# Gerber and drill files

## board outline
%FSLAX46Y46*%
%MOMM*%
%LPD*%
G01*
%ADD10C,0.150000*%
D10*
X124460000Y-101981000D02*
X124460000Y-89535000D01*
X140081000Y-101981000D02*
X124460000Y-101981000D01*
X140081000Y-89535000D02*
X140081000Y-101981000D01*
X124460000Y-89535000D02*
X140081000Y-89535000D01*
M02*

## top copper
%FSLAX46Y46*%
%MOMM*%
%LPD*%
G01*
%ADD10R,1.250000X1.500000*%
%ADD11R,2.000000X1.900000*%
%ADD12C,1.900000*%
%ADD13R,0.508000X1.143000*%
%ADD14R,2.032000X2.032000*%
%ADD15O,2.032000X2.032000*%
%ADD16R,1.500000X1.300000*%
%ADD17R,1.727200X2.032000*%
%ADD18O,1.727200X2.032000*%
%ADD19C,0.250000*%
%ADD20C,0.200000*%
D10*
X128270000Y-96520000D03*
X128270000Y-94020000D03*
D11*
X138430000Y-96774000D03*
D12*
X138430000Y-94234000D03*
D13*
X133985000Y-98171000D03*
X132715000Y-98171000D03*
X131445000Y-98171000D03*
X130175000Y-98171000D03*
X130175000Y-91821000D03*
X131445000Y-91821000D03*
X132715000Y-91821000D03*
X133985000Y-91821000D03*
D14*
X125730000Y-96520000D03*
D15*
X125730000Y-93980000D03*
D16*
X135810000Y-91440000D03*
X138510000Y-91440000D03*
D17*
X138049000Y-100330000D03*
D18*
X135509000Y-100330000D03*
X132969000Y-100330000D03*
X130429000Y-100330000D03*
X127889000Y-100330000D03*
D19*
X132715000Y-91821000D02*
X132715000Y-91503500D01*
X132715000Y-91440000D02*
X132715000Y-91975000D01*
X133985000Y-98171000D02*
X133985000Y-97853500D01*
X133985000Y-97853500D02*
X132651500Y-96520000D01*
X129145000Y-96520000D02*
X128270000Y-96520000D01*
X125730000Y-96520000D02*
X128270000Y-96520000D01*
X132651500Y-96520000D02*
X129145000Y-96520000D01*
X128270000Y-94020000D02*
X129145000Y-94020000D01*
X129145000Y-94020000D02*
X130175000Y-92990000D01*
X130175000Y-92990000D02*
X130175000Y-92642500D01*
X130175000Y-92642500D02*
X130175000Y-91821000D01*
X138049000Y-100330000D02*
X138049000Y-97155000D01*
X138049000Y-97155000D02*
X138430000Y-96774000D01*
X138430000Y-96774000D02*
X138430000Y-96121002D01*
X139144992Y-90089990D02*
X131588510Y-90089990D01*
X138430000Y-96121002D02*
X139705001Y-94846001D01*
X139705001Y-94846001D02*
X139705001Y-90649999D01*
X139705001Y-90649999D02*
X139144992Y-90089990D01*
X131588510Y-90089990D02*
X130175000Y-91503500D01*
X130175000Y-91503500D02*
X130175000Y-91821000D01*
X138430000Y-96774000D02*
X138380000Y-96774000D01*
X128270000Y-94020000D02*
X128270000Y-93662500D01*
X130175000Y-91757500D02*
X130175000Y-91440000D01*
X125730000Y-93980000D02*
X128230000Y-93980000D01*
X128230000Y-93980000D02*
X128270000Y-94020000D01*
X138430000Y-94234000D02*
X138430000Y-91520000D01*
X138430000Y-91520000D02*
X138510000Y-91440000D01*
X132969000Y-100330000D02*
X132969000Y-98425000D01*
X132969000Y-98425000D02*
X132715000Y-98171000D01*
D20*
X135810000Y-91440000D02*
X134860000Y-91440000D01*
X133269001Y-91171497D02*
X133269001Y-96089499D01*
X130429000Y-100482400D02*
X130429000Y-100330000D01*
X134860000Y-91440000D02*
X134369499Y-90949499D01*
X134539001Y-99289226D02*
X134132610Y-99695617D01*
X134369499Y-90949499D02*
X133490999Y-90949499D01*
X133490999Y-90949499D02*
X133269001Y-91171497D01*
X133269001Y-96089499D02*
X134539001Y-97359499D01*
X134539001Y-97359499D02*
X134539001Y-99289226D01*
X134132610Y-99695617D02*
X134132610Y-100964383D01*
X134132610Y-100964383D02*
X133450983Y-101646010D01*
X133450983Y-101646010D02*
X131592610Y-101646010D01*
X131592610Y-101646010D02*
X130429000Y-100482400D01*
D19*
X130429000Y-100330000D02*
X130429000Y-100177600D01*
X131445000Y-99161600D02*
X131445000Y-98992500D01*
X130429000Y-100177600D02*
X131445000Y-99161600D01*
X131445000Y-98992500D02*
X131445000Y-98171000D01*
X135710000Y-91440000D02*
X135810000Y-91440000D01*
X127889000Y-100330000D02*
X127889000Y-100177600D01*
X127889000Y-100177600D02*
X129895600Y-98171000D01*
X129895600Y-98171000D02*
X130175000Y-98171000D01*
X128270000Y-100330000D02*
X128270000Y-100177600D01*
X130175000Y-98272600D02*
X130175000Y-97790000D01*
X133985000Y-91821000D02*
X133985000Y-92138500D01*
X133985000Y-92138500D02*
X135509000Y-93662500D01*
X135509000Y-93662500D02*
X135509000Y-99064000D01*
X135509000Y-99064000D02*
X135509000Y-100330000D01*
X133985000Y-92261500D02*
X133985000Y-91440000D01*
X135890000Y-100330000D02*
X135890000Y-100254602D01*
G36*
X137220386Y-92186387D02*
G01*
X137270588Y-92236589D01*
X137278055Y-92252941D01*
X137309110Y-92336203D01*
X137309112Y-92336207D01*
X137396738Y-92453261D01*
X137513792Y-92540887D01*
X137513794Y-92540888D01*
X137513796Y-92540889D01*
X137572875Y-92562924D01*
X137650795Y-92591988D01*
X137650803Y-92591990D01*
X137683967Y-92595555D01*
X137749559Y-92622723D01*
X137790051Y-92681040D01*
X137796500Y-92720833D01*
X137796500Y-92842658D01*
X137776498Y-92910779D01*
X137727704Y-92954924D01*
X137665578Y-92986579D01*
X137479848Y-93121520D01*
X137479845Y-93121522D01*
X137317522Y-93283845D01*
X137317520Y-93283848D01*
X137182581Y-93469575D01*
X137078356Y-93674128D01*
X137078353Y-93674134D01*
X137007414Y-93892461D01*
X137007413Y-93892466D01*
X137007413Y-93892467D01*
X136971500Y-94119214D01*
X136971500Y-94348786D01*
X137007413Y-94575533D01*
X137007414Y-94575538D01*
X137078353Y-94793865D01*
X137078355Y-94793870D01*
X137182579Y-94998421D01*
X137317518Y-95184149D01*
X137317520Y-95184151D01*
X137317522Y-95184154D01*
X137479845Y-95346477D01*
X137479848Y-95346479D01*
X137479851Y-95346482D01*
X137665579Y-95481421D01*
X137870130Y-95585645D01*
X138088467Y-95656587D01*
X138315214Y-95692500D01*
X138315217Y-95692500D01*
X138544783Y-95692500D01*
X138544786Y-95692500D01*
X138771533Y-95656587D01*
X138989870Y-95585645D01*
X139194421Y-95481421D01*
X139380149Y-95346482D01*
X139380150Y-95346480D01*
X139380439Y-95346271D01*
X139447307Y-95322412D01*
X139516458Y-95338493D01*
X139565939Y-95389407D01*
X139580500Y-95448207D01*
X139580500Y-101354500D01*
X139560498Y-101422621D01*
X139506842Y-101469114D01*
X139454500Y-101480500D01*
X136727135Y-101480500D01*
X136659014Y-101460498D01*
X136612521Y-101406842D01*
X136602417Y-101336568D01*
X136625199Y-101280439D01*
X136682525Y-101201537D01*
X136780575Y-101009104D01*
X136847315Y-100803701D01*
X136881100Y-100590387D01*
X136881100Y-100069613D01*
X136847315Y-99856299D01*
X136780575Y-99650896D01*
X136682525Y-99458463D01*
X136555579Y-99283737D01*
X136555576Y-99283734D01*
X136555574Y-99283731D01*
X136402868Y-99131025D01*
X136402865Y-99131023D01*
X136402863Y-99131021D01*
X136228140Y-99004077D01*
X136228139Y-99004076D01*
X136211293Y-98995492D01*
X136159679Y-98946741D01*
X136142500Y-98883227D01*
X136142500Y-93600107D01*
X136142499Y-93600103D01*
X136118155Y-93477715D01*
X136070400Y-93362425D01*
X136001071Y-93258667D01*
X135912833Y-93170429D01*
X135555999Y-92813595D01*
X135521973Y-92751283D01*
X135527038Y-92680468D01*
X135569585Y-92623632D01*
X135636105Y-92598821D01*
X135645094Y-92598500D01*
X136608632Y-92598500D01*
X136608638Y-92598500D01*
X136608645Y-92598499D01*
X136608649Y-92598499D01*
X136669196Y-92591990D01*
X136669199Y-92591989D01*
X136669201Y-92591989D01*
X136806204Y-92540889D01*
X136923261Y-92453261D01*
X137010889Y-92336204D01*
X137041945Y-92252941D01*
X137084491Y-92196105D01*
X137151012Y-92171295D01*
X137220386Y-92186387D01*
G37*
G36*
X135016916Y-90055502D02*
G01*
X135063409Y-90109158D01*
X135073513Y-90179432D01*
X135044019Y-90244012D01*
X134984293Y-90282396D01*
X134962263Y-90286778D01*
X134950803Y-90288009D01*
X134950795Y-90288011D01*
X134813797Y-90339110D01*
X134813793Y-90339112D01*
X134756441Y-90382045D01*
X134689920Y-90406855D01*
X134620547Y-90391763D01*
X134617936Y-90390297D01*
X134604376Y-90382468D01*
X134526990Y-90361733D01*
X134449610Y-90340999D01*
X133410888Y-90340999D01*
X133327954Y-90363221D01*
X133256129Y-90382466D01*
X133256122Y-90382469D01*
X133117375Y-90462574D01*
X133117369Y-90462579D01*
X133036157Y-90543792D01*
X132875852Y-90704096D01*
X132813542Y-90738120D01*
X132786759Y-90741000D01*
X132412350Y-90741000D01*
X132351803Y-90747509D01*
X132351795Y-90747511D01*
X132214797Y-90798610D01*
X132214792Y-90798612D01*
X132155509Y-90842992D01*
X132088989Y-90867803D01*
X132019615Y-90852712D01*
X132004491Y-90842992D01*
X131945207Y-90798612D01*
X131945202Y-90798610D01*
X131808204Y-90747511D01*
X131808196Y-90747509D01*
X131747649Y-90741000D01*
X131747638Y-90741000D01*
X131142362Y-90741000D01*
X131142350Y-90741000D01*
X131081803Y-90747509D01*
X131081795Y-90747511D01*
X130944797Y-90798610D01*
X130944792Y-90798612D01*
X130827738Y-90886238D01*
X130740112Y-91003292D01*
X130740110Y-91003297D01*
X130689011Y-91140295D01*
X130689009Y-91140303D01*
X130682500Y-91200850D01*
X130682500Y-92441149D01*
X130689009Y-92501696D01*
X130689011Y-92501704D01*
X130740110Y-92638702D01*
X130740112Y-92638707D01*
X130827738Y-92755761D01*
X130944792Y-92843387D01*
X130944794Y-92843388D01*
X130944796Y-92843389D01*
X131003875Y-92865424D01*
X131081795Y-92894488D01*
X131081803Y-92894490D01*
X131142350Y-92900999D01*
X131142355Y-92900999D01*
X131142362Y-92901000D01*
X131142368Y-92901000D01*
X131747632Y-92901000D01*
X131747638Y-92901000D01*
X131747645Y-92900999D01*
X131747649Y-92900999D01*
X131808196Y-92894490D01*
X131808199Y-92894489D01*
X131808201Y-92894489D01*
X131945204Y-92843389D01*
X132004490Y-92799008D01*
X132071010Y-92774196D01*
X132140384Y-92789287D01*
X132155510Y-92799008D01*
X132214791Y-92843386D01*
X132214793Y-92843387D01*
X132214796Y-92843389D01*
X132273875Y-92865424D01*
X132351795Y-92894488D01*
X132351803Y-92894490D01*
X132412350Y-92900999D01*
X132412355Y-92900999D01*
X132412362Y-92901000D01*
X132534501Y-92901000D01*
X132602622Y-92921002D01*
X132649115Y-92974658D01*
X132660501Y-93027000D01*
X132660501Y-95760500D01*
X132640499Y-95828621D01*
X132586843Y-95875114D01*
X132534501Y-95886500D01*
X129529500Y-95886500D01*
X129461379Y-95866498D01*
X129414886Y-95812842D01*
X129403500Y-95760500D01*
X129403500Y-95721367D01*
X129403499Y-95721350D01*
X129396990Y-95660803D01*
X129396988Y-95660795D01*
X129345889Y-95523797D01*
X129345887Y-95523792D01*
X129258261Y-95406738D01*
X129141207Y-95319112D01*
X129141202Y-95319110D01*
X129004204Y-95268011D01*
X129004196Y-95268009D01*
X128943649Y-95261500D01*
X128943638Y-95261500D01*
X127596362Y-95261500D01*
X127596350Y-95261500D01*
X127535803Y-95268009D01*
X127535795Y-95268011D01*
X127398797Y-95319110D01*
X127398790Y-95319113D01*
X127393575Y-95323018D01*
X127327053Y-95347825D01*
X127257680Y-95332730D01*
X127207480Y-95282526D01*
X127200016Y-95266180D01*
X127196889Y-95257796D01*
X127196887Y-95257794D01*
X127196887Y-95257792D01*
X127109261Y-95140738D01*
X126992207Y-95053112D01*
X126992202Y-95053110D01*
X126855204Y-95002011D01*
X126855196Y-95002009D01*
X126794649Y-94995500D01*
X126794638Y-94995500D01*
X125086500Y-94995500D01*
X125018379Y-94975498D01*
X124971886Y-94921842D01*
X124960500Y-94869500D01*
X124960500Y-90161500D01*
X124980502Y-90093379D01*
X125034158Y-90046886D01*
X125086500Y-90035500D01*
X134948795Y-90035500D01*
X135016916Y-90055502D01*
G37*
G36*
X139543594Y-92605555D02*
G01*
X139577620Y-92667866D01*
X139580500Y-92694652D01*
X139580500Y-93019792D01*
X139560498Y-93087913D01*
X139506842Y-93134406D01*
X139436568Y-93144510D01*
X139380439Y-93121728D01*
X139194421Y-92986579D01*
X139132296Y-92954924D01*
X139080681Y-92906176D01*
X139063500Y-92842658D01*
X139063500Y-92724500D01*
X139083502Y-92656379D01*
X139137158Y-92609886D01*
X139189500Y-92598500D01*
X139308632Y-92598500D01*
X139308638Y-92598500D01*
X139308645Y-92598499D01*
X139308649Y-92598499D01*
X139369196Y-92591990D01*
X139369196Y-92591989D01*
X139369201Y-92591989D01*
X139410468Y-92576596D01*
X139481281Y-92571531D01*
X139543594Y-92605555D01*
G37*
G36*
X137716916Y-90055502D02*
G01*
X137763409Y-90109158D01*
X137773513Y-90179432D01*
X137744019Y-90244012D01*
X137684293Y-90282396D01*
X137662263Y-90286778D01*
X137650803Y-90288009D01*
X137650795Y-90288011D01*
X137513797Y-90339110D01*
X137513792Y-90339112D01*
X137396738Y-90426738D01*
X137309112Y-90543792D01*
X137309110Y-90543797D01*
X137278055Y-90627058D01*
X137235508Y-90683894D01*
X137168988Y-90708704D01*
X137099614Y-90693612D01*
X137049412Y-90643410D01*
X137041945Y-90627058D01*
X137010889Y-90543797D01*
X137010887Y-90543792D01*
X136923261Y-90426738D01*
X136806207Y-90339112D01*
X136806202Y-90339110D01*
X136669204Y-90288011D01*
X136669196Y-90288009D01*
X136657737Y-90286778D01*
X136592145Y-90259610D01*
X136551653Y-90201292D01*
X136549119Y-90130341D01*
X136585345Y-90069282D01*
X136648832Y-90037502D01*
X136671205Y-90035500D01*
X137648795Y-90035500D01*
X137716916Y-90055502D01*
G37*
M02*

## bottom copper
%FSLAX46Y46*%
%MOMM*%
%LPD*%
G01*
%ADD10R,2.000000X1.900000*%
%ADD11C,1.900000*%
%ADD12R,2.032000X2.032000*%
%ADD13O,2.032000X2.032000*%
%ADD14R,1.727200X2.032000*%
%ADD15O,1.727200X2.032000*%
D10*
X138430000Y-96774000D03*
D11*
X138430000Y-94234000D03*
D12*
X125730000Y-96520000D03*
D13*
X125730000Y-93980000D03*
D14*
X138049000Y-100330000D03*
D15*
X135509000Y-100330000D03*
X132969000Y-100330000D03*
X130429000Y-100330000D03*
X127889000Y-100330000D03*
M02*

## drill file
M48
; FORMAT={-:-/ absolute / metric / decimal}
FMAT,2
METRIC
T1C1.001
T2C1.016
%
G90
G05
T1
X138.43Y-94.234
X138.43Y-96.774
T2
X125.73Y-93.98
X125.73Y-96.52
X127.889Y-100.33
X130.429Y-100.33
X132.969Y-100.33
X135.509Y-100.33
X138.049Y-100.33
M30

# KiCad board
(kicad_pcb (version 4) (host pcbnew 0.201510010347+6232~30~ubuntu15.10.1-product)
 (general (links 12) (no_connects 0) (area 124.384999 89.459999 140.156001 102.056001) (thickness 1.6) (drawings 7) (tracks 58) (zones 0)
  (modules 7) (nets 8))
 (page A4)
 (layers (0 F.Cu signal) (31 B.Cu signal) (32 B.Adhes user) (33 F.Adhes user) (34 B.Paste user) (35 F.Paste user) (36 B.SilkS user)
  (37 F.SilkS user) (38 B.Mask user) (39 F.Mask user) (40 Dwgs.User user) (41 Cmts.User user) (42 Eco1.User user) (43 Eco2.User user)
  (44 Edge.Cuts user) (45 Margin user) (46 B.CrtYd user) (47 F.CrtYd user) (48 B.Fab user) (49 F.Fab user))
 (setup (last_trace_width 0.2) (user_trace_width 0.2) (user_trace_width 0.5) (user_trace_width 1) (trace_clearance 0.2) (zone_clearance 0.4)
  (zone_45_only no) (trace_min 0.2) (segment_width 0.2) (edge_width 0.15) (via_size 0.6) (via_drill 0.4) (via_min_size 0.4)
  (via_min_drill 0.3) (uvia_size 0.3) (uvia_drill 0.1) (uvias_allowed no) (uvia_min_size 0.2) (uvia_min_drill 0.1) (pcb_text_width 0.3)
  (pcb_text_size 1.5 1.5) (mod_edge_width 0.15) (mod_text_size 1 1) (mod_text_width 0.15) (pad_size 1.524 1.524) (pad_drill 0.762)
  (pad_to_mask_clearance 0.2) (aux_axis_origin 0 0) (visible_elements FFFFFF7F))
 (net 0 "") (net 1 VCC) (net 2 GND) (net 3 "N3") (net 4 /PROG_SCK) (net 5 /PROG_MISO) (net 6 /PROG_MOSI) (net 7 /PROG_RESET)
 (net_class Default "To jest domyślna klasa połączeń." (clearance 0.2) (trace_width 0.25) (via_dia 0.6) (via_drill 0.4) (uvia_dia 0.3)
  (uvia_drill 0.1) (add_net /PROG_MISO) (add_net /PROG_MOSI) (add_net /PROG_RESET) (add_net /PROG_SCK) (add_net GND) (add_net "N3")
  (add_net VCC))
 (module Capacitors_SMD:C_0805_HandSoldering (layer F.Cu) (at 128.27 95.27 90)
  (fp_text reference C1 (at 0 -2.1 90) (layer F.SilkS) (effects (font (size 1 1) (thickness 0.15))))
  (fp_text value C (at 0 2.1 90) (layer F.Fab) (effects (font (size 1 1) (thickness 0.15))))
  (pad 1 smd rect (at -1.25 0 90) (size 1.5 1.25) (layers F.Cu F.Paste F.Mask) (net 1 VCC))
  (pad 2 smd rect (at 1.25 0 90) (size 1.5 1.25) (layers F.Cu F.Paste F.Mask) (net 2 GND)))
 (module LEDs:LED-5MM (layer B.Cu) (at 138.43 96.774 90)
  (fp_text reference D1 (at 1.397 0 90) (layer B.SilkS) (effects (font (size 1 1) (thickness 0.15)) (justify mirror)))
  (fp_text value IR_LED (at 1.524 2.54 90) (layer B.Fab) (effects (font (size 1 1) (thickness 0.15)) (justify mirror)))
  (pad 1 thru_hole rect (at 0 0) (size 2 1.9) (drill 1.00076) (layers *.Cu *.Mask B.SilkS) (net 2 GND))
  (pad 2 thru_hole circle (at 2.54 0 90) (size 1.9 1.9) (drill 1.00076) (layers *.Cu *.Mask B.SilkS) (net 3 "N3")))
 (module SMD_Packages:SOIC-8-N (layer F.Cu) (at 132.08 94.996 180)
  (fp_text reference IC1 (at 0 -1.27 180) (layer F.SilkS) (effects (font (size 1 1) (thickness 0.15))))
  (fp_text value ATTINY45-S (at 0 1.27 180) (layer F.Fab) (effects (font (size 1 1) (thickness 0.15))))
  (pad 8 smd rect (at -1.905 -3.175 180) (size 0.508 1.143) (layers F.Cu F.Paste F.Mask) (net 1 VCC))
  (pad 7 smd rect (at -0.635 -3.175 180) (size 0.508 1.143) (layers F.Cu F.Paste F.Mask) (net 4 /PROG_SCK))
  (pad 6 smd rect (at 0.635 -3.175 180) (size 0.508 1.143) (layers F.Cu F.Paste F.Mask) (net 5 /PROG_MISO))
  (pad 5 smd rect (at 1.905 -3.175 180) (size 0.508 1.143) (layers F.Cu F.Paste F.Mask) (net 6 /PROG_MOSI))
  (pad 4 smd rect (at 1.905 3.175 180) (size 0.508 1.143) (layers F.Cu F.Paste F.Mask) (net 2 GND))
  (pad 3 smd rect (at 0.635 3.175 180) (size 0.508 1.143) (layers F.Cu F.Paste F.Mask))
  (pad 2 smd rect (at -0.635 3.175 180) (size 0.508 1.143) (layers F.Cu F.Paste F.Mask))
  (pad 1 smd rect (at -1.905 3.175 180) (size 0.508 1.143) (layers F.Cu F.Paste F.Mask) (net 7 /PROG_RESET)))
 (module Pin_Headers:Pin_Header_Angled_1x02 (layer F.Cu) (at 125.73 96.52 180)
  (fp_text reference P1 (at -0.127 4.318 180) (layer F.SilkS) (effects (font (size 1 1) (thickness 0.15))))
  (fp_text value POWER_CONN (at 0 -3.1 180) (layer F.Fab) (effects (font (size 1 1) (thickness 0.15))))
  (pad 1 thru_hole rect (at 0 0 180) (size 2.032 2.032) (drill 1.016) (layers *.Cu *.Mask F.SilkS) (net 1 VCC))
  (pad 2 thru_hole oval (at 0 2.54 180) (size 2.032 2.032) (drill 1.016) (layers *.Cu *.Mask F.SilkS) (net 2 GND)))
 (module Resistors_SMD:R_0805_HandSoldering (layer F.Cu) (at 137.16 91.44)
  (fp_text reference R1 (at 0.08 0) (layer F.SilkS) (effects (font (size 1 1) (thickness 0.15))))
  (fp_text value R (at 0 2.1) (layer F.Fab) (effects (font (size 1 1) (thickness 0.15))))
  (pad 1 smd rect (at -1.35 0) (size 1.5 1.3) (layers F.Cu F.Paste F.Mask) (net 5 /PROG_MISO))
  (pad 2 smd rect (at 1.35 0) (size 1.5 1.3) (layers F.Cu F.Paste F.Mask) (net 3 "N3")))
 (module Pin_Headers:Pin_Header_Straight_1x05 (layer F.Cu) (at 138.049 100.33 270)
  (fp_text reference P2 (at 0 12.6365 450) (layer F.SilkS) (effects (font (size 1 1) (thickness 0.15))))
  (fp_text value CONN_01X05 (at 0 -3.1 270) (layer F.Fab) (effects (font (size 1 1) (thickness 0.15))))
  (pad 1 thru_hole rect (at 0 0 270) (size 2.032 1.7272) (drill 1.016) (layers *.Cu *.Mask F.SilkS) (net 2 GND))
  (pad 2 thru_hole oval (at 0 2.54 270) (size 2.032 1.7272) (drill 1.016) (layers *.Cu *.Mask F.SilkS) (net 7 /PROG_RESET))
  (pad 3 thru_hole oval (at 0 5.08 270) (size 2.032 1.7272) (drill 1.016) (layers *.Cu *.Mask F.SilkS) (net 4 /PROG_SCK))
  (pad 4 thru_hole oval (at 0 7.62 270) (size 2.032 1.7272) (drill 1.016) (layers *.Cu *.Mask F.SilkS) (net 5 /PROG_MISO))
  (pad 5 thru_hole oval (at 0 10.16 270) (size 2.032 1.7272) (drill 1.016) (layers *.Cu *.Mask F.SilkS) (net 6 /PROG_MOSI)))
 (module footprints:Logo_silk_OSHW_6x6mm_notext (layer B.Cu) (at 129.794 92.202)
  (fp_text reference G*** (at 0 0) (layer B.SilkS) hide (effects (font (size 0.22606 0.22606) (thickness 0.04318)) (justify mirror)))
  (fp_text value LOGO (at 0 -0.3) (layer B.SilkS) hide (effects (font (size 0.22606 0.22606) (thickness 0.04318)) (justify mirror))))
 (gr_line (start 124.46 101.981) (end 124.46 89.535) (layer Edge.Cuts) (width 0.15))
 (gr_line (start 140.081 101.981) (end 124.46 101.981) (layer Edge.Cuts) (width 0.15))
 (gr_line (start 140.081 89.535) (end 140.081 101.981) (layer Edge.Cuts) (width 0.15))
 (gr_line (start 124.46 89.535) (end 140.081 89.535) (layer Edge.Cuts) (width 0.15))
 (segment (start 132.715 91.821) (end 132.715 91.5035) (width 0.25) (layer F.Cu) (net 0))
 (segment (start 132.715 91.44) (end 132.715 91.975) (width 0.25) (layer F.Cu) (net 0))
 (segment (start 133.985 98.171) (end 133.985 97.8535) (width 0.25) (layer F.Cu) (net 1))
 (segment (start 133.985 97.8535) (end 132.6515 96.52) (width 0.25) (layer F.Cu) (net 1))
 (segment (start 129.145 96.52) (end 128.27 96.52) (width 0.25) (layer F.Cu) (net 1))
 (segment (start 125.73 96.52) (end 128.27 96.52) (width 0.25) (layer F.Cu) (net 1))
 (segment (start 132.6515 96.52) (end 129.145 96.52) (width 0.25) (layer F.Cu) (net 1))
 (segment (start 128.27 94.02) (end 129.145 94.02) (width 0.25) (layer F.Cu) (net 2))
 (segment (start 129.145 94.02) (end 130.175 92.99) (width 0.25) (layer F.Cu) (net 2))
 (segment (start 130.175 92.99) (end 130.175 92.6425) (width 0.25) (layer F.Cu) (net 2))
 (segment (start 130.175 92.6425) (end 130.175 91.821) (width 0.25) (layer F.Cu) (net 2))
 (segment (start 138.049 100.33) (end 138.049 97.155) (width 0.25) (layer F.Cu) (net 2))
 (segment (start 138.049 97.155) (end 138.43 96.774) (width 0.25) (layer F.Cu) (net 2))
 (segment (start 138.43 96.774) (end 138.43 96.121002) (width 0.25) (layer F.Cu) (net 2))
 (segment (start 139.144992 90.08999) (end 131.58851 90.08999) (width 0.25) (layer F.Cu) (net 2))
 (segment (start 138.43 96.121002) (end 139.705001 94.846001) (width 0.25) (layer F.Cu) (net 2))
 (segment (start 139.705001 94.846001) (end 139.705001 90.649999) (width 0.25) (layer F.Cu) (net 2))
 (segment (start 139.705001 90.649999) (end 139.144992 90.08999) (width 0.25) (layer F.Cu) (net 2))
 (segment (start 131.58851 90.08999) (end 130.175 91.5035) (width 0.25) (layer F.Cu) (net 2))
 (segment (start 130.175 91.5035) (end 130.175 91.821) (width 0.25) (layer F.Cu) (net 2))
 (segment (start 138.43 96.774) (end 138.38 96.774) (width 0.25) (layer F.Cu) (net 2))
 (segment (start 128.27 94.02) (end 128.27 93.6625) (width 0.25) (layer F.Cu) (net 2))
 (segment (start 130.175 91.7575) (end 130.175 91.44) (width 0.25) (layer F.Cu) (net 2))
 (segment (start 125.73 93.98) (end 128.23 93.98) (width 0.25) (layer F.Cu) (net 2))
 (segment (start 128.23 93.98) (end 128.27 94.02) (width 0.25) (layer F.Cu) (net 2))
 (segment (start 138.43 94.234) (end 138.43 91.52) (width 0.25) (layer F.Cu) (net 3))
 (segment (start 138.43 91.52) (end 138.51 91.44) (width 0.25) (layer F.Cu) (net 3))
 (segment (start 132.969 100.33) (end 132.969 98.425) (width 0.25) (layer F.Cu) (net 4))
 (segment (start 132.969 98.425) (end 132.715 98.171) (width 0.25) (layer F.Cu) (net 4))
 (segment (start 135.81 91.44) (end 134.86 91.44) (width 0.2) (layer F.Cu) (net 5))
 (segment (start 133.269001 91.171497) (end 133.269001 96.089499) (width 0.2) (layer F.Cu) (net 5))
 (segment (start 130.429 100.4824) (end 130.429 100.33) (width 0.2) (layer F.Cu) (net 5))
 (segment (start 134.86 91.44) (end 134.369499 90.949499) (width 0.2) (layer F.Cu) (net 5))
 (segment (start 134.539001 99.289226) (end 134.13261 99.695617) (width 0.2) (layer F.Cu) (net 5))
 (segment (start 134.369499 90.949499) (end 133.490999 90.949499) (width 0.2) (layer F.Cu) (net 5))
 (segment (start 133.490999 90.949499) (end 133.269001 91.171497) (width 0.2) (layer F.Cu) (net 5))
 (segment (start 133.269001 96.089499) (end 134.539001 97.359499) (width 0.2) (layer F.Cu) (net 5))
 (segment (start 134.539001 97.359499) (end 134.539001 99.289226) (width 0.2) (layer F.Cu) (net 5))
 (segment (start 134.13261 99.695617) (end 134.13261 100.964383) (width 0.2) (layer F.Cu) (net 5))
 (segment (start 134.13261 100.964383) (end 133.450983 101.64601) (width 0.2) (layer F.Cu) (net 5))
 (segment (start 133.450983 101.64601) (end 131.59261 101.64601) (width 0.2) (layer F.Cu) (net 5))
 (segment (start 131.59261 101.64601) (end 130.429 100.4824) (width 0.2) (layer F.Cu) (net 5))
 (segment (start 130.429 100.33) (end 130.429 100.1776) (width 0.25) (layer F.Cu) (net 5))
 (segment (start 131.445 99.1616) (end 131.445 98.9925) (width 0.25) (layer F.Cu) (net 5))
 (segment (start 130.429 100.1776) (end 131.445 99.1616) (width 0.25) (layer F.Cu) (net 5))
 (segment (start 131.445 98.9925) (end 131.445 98.171) (width 0.25) (layer F.Cu) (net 5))
 (segment (start 135.71 91.44) (end 135.81 91.44) (width 0.25) (layer F.Cu) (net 5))
 (segment (start 127.889 100.33) (end 127.889 100.1776) (width 0.25) (layer F.Cu) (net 6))
 (segment (start 127.889 100.1776) (end 129.8956 98.171) (width 0.25) (layer F.Cu) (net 6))
 (segment (start 129.8956 98.171) (end 130.175 98.171) (width 0.25) (layer F.Cu) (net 6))
 (segment (start 128.27 100.33) (end 128.27 100.1776) (width 0.25) (layer F.Cu) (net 6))
 (segment (start 130.175 98.2726) (end 130.175 97.79) (width 0.25) (layer F.Cu) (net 6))
 (segment (start 133.985 91.821) (end 133.985 92.1385) (width 0.25) (layer F.Cu) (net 7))
 (segment (start 133.985 92.1385) (end 135.509 93.6625) (width 0.25) (layer F.Cu) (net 7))
 (segment (start 135.509 93.6625) (end 135.509 99.064) (width 0.25) (layer F.Cu) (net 7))
 (segment (start 135.509 99.064) (end 135.509 100.33) (width 0.25) (layer F.Cu) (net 7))
 (segment (start 133.985 92.2615) (end 133.985 91.44) (width 0.25) (layer F.Cu) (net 7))
 (segment (start 135.89 100.33) (end 135.89 100.254602) (width 0.25) (layer F.Cu) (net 7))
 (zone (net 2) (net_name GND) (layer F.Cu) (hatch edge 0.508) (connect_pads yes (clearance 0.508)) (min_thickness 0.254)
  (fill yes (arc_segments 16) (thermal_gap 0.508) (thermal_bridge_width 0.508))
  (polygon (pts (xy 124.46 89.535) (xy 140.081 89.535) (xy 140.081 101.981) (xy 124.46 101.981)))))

